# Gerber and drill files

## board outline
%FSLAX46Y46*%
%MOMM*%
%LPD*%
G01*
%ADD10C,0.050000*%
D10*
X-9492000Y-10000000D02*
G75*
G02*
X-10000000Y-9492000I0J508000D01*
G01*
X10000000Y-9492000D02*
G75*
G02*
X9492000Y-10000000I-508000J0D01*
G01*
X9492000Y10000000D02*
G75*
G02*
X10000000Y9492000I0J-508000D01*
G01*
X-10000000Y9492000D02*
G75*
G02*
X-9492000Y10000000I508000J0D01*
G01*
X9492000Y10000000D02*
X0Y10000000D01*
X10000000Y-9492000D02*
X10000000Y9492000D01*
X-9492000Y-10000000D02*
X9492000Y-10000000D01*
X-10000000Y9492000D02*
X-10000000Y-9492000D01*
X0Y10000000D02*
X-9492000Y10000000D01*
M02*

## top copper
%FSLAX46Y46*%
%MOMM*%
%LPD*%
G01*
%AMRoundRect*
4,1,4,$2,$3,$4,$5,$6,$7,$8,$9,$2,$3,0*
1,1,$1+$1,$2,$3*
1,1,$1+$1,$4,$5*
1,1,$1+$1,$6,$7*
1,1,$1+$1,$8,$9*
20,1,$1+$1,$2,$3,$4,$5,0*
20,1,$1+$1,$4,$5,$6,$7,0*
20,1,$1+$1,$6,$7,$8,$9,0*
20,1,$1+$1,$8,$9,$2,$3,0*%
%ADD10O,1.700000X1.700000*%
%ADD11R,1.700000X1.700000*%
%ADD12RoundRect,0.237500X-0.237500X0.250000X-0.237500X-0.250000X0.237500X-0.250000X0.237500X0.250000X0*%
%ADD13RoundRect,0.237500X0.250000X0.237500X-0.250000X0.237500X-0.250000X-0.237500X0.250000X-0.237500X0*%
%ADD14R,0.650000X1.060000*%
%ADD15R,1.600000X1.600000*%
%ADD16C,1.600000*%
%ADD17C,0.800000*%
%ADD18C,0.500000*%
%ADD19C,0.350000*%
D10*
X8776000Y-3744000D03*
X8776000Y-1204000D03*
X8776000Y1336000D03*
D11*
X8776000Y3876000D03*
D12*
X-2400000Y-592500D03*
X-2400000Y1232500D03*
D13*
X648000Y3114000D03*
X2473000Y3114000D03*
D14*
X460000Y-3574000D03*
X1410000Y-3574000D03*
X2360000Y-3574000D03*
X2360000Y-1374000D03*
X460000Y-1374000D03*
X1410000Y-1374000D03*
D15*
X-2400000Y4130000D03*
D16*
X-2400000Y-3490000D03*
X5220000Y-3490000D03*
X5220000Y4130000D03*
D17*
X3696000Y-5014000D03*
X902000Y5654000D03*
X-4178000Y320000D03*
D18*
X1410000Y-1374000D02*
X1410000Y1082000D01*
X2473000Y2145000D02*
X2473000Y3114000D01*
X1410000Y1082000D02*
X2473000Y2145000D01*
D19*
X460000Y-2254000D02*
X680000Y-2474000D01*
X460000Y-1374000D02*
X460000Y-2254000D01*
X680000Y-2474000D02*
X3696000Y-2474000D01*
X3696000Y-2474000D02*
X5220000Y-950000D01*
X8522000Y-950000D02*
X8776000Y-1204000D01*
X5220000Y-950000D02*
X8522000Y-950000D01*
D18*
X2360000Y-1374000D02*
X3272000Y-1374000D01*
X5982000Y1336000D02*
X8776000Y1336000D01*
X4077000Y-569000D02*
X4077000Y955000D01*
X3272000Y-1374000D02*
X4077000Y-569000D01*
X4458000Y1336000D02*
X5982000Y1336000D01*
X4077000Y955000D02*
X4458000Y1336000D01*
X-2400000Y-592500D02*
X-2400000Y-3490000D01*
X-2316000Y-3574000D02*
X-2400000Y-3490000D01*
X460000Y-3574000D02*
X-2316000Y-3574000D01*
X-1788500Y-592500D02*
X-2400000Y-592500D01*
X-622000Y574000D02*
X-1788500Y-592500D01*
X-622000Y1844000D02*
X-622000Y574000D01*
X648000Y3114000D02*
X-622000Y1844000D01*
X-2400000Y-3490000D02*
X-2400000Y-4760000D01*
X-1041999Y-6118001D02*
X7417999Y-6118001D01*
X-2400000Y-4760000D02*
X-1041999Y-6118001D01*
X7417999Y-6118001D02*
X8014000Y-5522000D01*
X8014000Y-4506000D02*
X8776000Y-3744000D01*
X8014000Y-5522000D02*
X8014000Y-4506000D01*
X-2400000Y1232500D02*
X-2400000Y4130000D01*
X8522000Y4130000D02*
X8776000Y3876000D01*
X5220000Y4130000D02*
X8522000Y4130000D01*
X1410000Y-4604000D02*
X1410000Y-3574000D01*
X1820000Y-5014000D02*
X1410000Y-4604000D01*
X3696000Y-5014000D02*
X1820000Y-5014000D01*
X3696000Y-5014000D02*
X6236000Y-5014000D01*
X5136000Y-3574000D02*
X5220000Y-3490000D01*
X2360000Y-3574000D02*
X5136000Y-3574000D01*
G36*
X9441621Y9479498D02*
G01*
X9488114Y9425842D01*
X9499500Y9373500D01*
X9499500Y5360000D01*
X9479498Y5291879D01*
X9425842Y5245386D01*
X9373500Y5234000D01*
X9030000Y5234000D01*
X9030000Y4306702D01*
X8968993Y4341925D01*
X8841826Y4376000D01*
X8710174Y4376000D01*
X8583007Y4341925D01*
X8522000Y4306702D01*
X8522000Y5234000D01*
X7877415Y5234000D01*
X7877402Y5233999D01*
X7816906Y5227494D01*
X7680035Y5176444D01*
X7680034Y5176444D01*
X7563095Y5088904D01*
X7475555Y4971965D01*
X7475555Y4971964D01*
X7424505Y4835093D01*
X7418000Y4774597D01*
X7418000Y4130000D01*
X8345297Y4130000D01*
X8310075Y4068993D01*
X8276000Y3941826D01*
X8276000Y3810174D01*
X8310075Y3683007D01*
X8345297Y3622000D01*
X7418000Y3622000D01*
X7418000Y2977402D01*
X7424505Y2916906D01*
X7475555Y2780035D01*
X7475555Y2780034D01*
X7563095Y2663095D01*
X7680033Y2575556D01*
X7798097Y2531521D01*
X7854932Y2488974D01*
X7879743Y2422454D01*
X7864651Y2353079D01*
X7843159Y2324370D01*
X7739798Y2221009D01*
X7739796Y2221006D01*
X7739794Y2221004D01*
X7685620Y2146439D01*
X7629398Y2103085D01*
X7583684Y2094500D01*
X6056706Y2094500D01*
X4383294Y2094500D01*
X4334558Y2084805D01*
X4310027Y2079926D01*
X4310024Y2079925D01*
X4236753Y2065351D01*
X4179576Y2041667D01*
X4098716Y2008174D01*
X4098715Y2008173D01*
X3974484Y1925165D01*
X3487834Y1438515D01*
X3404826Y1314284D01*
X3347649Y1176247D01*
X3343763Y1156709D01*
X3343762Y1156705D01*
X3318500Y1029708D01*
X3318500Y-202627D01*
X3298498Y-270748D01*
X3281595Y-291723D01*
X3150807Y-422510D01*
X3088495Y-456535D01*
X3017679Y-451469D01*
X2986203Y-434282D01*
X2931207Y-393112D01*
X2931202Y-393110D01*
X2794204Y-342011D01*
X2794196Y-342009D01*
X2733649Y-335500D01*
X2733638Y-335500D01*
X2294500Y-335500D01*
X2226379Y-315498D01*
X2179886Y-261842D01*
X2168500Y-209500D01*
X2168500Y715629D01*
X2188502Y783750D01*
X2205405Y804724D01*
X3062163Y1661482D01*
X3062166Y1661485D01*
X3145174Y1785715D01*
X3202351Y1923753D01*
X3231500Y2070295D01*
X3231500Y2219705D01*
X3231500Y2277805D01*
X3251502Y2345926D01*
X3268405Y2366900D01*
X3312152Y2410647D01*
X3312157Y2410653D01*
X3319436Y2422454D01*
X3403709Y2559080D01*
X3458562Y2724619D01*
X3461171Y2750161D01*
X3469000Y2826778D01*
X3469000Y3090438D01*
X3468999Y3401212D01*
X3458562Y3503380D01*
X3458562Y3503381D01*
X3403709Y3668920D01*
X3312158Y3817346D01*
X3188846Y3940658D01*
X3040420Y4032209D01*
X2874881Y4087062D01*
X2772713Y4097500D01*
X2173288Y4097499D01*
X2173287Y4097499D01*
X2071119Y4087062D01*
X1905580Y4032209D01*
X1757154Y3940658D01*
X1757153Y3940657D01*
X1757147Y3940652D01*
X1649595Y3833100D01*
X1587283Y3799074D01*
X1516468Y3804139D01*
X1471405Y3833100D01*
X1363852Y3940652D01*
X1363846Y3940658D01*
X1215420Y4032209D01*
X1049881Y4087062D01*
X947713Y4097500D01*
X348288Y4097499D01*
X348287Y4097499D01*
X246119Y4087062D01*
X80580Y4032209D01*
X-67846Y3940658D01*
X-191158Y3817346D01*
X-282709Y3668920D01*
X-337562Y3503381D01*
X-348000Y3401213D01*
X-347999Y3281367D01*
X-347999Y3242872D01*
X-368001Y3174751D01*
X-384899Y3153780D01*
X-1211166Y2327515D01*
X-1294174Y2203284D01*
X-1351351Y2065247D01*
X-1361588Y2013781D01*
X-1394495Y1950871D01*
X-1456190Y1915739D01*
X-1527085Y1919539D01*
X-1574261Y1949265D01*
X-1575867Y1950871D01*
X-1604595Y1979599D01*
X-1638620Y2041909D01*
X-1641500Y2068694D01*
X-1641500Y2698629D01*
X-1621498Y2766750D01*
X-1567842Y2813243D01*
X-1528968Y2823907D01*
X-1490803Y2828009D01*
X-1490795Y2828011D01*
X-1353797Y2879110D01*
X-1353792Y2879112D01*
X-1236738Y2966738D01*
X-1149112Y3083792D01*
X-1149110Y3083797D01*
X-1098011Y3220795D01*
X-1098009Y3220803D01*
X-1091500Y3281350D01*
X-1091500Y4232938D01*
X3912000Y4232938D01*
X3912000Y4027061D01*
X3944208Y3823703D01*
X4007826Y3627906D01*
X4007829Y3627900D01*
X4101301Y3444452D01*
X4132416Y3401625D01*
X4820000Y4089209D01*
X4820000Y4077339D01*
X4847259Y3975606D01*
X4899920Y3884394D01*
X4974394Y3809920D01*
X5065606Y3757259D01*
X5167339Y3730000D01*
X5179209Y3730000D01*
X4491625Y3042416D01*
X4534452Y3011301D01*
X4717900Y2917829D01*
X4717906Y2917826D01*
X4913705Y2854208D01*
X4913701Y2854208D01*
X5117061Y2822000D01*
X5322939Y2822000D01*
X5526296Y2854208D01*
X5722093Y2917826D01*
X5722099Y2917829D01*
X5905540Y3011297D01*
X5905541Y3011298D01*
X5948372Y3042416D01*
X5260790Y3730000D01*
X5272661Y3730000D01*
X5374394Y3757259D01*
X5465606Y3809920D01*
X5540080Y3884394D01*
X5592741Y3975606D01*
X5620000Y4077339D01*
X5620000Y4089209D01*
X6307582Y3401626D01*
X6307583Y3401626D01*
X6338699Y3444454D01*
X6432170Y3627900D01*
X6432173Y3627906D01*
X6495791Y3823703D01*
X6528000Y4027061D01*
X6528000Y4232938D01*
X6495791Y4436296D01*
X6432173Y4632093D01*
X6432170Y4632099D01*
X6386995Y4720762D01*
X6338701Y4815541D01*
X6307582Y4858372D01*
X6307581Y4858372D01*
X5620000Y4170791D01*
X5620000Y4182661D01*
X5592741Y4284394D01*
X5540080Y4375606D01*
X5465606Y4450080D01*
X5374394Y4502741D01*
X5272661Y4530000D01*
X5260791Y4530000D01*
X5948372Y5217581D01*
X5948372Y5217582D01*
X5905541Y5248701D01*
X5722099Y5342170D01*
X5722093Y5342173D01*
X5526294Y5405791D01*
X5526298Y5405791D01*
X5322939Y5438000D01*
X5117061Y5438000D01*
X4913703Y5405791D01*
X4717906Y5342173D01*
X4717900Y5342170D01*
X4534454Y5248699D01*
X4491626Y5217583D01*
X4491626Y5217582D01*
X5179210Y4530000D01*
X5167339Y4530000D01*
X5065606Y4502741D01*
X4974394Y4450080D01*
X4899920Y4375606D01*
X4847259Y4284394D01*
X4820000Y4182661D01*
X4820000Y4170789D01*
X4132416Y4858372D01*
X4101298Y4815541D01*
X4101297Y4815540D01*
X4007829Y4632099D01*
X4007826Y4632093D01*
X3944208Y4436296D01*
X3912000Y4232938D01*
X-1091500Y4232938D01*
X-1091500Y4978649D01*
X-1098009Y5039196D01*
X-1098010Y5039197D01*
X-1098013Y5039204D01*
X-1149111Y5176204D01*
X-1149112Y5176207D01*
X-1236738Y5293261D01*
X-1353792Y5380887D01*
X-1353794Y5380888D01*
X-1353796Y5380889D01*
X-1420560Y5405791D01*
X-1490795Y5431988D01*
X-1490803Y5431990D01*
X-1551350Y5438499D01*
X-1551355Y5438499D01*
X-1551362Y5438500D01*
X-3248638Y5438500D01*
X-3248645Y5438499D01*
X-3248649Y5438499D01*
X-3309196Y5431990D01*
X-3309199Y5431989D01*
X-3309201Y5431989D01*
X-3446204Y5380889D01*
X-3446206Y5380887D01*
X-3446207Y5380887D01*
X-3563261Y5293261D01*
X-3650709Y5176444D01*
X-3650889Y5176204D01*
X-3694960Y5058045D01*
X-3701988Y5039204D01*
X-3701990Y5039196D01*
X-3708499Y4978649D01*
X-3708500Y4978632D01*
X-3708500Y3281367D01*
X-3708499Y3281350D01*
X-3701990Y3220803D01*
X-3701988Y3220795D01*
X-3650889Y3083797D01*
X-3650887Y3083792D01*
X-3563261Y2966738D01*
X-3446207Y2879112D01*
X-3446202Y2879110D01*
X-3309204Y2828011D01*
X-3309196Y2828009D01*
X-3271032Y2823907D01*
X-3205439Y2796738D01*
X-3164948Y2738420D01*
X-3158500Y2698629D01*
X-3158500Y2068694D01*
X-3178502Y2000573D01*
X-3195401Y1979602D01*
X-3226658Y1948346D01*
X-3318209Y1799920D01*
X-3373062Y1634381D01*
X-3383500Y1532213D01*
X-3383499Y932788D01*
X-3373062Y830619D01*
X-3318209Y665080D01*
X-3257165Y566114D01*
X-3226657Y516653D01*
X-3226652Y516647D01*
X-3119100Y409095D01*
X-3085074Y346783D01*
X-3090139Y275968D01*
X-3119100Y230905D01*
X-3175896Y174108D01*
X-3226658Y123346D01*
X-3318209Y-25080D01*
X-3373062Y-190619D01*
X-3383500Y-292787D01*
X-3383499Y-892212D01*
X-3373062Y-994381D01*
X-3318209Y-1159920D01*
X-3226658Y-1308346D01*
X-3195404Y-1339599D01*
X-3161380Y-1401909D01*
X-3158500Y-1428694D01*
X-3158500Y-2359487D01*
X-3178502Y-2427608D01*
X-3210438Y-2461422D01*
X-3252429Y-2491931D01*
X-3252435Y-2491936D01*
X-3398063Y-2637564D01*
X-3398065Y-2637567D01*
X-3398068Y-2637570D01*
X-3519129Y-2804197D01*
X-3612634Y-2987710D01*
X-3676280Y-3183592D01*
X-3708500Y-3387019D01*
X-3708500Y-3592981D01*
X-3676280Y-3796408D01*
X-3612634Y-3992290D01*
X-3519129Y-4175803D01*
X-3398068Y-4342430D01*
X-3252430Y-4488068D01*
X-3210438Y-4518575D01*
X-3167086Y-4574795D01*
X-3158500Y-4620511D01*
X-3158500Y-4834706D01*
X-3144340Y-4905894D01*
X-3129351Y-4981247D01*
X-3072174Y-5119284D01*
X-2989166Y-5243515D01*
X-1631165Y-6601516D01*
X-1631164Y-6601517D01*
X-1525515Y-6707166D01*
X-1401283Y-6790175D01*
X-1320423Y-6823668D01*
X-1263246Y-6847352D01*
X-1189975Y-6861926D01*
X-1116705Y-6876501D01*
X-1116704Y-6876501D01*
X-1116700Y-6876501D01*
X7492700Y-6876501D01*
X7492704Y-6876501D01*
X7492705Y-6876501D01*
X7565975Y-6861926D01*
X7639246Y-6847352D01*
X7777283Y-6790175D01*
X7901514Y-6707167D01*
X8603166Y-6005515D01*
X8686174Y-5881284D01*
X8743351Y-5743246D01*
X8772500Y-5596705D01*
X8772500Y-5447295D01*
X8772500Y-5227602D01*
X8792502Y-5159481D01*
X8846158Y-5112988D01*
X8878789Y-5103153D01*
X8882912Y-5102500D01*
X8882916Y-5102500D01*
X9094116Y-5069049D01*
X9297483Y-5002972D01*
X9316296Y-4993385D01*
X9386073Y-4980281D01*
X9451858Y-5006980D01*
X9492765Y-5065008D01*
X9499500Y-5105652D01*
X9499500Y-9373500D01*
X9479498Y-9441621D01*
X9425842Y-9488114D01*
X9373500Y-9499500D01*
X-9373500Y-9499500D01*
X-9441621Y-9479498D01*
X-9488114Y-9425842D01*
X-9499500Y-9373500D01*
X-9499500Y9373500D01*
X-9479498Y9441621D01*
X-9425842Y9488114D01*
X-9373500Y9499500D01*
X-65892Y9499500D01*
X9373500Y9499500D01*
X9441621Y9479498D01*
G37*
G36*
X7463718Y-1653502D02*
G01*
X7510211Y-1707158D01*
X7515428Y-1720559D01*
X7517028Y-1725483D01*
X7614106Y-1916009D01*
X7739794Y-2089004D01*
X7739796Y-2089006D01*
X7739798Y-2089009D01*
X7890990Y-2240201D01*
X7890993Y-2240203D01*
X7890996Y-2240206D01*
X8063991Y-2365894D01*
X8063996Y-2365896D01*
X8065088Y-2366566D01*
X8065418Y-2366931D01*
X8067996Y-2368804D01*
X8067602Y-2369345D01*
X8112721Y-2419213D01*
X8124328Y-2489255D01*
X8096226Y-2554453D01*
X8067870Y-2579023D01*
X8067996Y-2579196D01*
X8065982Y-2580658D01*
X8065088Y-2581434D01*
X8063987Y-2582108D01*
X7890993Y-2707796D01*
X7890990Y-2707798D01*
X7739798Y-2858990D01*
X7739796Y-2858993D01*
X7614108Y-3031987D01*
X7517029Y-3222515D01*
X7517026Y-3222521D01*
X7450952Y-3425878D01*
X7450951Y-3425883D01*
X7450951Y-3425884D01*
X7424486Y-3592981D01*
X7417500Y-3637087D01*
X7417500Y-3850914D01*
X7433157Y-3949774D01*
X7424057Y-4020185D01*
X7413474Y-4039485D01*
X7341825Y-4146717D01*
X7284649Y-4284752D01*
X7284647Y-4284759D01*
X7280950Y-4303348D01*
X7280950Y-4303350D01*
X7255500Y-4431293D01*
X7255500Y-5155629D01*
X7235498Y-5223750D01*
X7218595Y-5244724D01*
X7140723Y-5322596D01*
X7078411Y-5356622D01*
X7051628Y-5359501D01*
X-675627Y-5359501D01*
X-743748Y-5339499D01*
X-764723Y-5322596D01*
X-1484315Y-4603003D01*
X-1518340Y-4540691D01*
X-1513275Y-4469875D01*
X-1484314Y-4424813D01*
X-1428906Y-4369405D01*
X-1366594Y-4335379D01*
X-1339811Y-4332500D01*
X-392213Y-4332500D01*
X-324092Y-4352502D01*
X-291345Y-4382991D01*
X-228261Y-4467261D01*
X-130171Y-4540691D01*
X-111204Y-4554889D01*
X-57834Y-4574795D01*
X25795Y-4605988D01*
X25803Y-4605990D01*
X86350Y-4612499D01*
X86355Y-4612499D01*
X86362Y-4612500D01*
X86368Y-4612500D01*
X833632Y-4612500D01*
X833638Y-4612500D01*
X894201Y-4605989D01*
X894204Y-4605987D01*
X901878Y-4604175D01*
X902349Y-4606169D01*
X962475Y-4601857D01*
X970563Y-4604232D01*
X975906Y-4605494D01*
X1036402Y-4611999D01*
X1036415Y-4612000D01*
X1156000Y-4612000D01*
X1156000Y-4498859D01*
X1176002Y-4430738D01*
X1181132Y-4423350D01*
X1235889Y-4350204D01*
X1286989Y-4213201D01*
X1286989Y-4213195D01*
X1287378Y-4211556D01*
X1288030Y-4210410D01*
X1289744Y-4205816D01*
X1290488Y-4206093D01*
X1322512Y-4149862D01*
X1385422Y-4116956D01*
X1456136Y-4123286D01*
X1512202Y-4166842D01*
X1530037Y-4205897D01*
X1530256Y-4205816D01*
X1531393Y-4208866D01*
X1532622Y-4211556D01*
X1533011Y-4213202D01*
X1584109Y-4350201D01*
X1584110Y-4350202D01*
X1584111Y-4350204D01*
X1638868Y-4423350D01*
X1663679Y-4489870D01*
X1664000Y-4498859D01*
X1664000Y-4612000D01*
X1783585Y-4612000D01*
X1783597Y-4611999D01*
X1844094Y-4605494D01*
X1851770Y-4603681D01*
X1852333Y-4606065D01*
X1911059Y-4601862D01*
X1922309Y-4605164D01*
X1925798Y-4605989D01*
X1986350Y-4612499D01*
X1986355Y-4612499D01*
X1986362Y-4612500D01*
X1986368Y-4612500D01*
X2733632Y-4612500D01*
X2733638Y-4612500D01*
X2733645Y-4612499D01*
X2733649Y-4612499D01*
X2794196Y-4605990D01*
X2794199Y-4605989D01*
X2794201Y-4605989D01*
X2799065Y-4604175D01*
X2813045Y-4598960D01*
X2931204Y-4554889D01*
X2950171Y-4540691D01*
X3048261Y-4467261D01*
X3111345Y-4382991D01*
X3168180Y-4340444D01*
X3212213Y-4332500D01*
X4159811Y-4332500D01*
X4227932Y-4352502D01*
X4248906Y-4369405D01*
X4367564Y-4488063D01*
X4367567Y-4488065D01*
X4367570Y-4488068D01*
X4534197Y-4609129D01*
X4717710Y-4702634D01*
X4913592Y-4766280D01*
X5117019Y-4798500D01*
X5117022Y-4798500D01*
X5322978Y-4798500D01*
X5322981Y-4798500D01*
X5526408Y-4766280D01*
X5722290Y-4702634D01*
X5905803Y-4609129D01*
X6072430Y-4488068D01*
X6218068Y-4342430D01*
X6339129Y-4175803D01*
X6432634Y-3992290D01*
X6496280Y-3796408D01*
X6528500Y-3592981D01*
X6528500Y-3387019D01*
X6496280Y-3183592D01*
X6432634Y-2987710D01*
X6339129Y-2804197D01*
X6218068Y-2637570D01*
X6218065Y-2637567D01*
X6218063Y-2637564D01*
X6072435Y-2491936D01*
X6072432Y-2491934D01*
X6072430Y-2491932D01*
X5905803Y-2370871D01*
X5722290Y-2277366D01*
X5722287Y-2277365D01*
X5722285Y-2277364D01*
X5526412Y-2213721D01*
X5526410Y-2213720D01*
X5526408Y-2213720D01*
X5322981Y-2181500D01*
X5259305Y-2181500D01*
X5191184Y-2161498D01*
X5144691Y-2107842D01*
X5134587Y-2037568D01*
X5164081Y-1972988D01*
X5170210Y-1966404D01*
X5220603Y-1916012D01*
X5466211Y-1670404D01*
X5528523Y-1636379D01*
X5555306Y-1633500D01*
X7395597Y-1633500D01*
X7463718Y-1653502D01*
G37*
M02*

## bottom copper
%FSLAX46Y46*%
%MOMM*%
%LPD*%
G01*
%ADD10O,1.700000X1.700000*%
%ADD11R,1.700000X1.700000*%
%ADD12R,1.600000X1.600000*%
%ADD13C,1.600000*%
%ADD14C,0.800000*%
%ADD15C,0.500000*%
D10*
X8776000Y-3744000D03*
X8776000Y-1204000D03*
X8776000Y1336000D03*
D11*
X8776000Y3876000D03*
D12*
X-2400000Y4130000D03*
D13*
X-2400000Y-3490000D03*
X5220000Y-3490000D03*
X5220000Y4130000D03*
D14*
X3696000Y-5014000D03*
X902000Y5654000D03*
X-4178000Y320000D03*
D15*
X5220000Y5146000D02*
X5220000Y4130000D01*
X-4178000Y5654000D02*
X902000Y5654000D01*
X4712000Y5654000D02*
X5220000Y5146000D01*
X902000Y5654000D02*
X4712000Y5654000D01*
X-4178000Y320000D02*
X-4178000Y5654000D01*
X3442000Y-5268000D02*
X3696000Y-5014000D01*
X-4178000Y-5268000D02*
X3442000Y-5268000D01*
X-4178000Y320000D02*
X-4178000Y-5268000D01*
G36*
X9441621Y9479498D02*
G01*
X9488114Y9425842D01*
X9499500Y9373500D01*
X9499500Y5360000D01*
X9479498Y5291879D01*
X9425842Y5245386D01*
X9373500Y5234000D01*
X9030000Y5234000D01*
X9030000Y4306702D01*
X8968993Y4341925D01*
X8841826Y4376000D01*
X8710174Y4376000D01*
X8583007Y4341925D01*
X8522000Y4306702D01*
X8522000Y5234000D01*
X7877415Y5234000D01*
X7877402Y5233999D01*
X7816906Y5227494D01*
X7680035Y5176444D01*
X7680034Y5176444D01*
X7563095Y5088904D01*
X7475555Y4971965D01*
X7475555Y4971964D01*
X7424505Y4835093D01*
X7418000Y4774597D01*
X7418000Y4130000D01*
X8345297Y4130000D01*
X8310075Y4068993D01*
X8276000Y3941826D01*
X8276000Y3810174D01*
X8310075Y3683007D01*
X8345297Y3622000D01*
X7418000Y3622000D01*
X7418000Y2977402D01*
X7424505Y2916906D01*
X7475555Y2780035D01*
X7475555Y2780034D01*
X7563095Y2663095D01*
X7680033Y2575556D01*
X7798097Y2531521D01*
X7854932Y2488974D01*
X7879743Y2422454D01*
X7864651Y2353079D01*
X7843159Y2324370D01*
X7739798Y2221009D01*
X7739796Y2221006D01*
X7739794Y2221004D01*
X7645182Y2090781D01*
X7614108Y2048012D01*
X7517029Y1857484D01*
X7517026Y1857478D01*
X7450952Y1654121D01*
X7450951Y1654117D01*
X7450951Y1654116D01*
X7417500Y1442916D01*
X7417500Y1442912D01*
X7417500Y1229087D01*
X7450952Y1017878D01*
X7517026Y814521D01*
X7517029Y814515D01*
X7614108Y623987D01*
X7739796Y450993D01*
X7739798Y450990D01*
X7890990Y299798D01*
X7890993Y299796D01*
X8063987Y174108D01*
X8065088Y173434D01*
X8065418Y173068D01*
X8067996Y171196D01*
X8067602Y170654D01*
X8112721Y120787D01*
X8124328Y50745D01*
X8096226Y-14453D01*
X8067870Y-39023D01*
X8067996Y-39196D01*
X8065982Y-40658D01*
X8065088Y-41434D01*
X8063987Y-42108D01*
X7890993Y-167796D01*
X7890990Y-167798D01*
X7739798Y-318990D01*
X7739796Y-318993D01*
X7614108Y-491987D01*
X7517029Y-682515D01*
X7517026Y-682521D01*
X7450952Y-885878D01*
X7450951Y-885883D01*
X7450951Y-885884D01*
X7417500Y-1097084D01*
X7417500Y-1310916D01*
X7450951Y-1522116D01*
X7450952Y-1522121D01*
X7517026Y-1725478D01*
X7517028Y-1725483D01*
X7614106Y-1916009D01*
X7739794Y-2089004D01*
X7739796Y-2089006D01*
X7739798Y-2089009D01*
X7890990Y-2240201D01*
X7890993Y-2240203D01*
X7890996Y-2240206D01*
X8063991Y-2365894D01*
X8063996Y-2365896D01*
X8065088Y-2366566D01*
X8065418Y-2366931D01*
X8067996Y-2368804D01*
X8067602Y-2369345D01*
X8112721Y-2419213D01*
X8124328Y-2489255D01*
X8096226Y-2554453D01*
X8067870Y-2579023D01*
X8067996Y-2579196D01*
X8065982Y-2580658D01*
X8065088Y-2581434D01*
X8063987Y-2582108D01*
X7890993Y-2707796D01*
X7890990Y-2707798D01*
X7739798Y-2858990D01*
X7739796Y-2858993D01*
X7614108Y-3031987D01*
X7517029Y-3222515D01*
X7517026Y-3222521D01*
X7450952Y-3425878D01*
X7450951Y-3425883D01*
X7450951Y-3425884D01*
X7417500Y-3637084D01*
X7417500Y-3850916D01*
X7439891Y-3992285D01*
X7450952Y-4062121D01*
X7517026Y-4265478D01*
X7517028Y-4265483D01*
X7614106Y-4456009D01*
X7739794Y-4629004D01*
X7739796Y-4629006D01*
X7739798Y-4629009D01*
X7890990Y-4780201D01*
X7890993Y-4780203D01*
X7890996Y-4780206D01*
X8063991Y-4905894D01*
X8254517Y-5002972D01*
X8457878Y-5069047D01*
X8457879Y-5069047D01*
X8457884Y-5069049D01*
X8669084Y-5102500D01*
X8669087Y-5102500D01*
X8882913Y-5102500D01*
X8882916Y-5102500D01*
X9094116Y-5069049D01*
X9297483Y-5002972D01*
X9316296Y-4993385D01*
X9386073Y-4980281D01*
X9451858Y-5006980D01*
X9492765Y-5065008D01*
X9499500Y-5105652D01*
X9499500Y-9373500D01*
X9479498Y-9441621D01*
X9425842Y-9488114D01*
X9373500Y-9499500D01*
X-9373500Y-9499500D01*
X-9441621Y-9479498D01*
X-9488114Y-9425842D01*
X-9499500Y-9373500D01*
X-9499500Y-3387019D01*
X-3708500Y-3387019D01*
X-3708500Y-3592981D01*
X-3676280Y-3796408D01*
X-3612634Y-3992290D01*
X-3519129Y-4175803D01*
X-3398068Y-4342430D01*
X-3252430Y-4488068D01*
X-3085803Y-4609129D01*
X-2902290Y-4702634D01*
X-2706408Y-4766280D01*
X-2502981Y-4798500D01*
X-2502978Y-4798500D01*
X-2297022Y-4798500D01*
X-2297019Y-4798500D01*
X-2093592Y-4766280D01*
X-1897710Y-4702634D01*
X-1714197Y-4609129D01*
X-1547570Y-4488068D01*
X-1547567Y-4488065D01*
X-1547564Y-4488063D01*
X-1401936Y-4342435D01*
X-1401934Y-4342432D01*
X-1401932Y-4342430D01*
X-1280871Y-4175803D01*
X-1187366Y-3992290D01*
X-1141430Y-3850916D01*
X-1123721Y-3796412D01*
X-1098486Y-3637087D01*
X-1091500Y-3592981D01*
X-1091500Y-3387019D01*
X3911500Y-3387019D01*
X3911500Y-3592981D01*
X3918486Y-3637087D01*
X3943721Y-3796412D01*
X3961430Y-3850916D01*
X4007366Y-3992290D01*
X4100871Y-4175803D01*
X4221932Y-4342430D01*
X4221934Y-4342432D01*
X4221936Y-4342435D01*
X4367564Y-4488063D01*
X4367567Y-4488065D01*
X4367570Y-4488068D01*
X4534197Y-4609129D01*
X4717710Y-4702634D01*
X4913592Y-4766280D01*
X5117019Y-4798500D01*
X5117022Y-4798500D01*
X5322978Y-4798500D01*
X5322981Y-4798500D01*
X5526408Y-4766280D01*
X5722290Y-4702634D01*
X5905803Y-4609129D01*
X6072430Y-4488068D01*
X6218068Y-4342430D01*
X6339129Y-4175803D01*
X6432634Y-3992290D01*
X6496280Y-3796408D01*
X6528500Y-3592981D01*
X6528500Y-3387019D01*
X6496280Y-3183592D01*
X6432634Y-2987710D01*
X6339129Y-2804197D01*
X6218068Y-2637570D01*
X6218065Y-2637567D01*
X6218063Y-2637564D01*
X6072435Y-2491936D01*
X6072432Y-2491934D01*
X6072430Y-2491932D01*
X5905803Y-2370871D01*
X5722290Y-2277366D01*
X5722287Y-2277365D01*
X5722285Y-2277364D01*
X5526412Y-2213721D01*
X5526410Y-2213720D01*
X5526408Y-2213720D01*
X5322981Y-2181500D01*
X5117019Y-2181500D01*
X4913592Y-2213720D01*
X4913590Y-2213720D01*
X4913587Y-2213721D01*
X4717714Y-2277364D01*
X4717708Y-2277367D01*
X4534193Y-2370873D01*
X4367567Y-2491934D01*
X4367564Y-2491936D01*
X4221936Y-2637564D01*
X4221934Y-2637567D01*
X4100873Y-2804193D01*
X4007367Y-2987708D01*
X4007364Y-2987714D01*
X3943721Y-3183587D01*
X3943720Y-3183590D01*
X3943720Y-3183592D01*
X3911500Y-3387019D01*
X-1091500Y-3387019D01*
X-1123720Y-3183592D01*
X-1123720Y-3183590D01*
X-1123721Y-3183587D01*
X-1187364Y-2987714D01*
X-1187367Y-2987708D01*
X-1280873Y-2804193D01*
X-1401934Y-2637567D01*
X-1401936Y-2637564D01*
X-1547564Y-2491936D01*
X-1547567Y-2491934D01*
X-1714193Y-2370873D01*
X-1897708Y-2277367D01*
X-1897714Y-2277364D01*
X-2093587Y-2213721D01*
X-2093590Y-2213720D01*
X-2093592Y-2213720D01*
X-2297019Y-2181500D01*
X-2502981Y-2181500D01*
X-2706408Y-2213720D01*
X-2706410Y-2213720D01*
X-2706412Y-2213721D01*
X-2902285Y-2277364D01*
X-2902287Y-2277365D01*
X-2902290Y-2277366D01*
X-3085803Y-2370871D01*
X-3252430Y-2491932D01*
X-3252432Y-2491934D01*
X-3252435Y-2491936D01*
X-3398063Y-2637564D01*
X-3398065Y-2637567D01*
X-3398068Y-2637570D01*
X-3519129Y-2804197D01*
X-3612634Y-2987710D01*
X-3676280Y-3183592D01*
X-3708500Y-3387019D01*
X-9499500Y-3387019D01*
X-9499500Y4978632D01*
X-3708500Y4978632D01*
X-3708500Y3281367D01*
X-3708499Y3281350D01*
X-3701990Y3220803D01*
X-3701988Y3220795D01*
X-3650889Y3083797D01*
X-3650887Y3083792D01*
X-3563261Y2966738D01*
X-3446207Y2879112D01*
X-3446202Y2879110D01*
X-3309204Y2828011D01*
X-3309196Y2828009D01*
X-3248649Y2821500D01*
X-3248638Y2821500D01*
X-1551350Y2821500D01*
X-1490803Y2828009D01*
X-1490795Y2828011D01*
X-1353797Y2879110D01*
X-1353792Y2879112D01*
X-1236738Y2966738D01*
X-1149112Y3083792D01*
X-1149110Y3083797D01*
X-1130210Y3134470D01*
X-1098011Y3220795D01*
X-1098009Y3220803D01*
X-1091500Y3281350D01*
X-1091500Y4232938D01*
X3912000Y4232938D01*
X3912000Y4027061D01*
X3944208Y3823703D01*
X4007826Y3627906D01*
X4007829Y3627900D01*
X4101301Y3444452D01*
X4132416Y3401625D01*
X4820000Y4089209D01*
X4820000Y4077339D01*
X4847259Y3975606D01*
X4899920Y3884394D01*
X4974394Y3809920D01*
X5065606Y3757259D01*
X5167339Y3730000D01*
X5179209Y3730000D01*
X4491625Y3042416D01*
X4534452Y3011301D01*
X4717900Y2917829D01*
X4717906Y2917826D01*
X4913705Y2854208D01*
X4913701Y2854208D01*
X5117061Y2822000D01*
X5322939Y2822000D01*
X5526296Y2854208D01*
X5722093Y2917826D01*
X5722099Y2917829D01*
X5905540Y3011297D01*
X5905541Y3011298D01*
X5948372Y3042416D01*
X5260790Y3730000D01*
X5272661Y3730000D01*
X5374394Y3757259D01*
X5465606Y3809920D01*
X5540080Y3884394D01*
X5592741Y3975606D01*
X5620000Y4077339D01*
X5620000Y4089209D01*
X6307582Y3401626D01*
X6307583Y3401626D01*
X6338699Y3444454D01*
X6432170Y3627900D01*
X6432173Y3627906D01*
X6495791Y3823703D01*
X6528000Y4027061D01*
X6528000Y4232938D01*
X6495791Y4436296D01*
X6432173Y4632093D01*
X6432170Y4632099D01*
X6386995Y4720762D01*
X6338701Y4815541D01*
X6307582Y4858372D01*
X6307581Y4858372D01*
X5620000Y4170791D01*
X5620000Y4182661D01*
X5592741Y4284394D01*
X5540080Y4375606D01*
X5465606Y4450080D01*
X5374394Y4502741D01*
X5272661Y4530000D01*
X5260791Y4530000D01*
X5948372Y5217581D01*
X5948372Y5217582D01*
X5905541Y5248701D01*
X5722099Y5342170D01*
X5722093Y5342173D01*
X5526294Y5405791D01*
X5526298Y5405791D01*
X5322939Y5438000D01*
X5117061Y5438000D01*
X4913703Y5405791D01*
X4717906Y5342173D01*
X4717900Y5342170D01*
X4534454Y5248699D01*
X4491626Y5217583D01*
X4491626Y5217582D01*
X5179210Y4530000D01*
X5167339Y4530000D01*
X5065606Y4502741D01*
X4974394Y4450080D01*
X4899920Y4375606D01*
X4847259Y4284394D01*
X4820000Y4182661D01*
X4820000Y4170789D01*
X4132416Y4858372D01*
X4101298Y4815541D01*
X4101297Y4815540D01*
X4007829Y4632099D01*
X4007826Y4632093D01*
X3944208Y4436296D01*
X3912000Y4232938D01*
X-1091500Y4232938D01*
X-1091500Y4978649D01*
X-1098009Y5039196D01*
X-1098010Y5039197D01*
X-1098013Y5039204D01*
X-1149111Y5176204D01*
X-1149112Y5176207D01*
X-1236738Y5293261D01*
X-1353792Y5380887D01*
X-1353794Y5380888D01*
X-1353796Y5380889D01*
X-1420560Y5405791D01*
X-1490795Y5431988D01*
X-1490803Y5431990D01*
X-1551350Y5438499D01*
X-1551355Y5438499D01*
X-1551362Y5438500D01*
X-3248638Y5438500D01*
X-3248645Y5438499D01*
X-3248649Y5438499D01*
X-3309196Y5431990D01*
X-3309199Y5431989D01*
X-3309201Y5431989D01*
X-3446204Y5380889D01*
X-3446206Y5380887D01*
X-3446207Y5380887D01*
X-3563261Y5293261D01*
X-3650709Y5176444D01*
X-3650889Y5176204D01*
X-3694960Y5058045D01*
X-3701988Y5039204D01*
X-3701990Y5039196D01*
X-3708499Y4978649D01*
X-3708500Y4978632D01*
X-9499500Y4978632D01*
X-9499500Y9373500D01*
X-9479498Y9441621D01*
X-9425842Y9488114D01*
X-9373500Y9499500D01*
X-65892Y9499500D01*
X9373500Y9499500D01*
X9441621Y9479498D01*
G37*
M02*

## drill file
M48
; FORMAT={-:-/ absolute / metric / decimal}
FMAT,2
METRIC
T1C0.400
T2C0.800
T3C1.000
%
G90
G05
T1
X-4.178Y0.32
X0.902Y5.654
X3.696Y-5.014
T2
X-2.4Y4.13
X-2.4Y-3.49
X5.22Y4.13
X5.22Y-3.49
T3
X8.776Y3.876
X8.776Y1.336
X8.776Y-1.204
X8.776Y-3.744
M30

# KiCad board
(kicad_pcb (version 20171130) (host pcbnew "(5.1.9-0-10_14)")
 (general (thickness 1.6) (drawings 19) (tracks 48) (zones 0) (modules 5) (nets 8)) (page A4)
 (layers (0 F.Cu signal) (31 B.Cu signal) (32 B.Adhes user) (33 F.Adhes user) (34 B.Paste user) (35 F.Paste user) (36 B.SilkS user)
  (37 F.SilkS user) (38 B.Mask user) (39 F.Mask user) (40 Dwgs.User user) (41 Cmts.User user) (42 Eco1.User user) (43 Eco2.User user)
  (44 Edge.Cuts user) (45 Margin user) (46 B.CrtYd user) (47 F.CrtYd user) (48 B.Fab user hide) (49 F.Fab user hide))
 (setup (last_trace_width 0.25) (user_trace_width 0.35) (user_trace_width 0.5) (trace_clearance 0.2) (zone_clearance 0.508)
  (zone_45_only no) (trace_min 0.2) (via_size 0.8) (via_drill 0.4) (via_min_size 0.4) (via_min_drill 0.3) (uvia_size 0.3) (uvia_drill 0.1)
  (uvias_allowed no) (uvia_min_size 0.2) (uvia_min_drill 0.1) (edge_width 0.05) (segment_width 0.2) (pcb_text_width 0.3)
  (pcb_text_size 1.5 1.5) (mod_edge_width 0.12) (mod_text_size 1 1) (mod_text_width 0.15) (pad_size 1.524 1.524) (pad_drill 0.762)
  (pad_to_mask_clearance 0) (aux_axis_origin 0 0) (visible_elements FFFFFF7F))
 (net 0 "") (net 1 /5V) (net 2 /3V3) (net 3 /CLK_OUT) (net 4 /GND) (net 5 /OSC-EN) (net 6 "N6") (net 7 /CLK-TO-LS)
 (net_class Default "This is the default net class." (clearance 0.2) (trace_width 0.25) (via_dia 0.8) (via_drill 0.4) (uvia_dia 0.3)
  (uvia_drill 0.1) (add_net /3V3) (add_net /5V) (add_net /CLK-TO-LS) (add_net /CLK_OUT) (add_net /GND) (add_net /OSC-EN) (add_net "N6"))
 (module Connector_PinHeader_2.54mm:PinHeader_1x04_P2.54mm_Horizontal (layer F.Cu) (at 8.776 -3.876)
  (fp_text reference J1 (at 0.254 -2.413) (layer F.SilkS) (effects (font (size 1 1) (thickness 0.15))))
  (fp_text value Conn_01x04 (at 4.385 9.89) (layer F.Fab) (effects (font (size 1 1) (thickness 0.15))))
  (pad 4 thru_hole oval (at 0 7.62) (size 1.7 1.7) (drill 1) (layers *.Cu *.Mask) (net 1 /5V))
  (pad 3 thru_hole oval (at 0 5.08) (size 1.7 1.7) (drill 1) (layers *.Cu *.Mask) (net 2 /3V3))
  (pad 2 thru_hole oval (at 0 2.54) (size 1.7 1.7) (drill 1) (layers *.Cu *.Mask) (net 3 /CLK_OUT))
  (pad 1 thru_hole rect (at 0 0) (size 1.7 1.7) (drill 1) (layers *.Cu *.Mask) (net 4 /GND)))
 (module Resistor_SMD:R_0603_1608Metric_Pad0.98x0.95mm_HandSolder (layer F.Cu) (at -2.4 -0.32 270)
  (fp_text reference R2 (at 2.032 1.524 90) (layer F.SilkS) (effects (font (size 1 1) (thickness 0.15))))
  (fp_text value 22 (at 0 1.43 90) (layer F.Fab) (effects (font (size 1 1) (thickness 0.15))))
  (pad 2 smd roundrect (at 0.9125 0 270) (size 0.975 0.95) (layers F.Cu F.Paste F.Mask) (roundrect_rratio 0.25) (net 1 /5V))
  (pad 1 smd roundrect (at -0.9125 0 270) (size 0.975 0.95) (layers F.Cu F.Paste F.Mask) (roundrect_rratio 0.25) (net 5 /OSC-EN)))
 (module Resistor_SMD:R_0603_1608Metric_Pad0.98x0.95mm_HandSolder (layer F.Cu) (at 1.5605 -3.114 180)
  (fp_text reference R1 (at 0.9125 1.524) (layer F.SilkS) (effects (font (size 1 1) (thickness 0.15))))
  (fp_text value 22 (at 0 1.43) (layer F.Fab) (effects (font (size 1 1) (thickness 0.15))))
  (pad 2 smd roundrect (at 0.9125 0 180) (size 0.975 0.95) (layers F.Cu F.Paste F.Mask) (roundrect_rratio 0.25) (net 1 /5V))
  (pad 1 smd roundrect (at -0.9125 0 180) (size 0.975 0.95) (layers F.Cu F.Paste F.Mask) (roundrect_rratio 0.25) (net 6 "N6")))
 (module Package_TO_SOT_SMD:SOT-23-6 (layer F.Cu) (at 1.41 2.474 90)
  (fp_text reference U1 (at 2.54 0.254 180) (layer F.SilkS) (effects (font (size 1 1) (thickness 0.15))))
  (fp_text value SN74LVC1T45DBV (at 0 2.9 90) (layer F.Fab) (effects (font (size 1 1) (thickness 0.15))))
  (pad 1 smd rect (at -1.1 -0.95 90) (size 1.06 0.65) (layers F.Cu F.Paste F.Mask) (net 1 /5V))
  (pad 2 smd rect (at -1.1 0 90) (size 1.06 0.65) (layers F.Cu F.Paste F.Mask) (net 4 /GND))
  (pad 3 smd rect (at -1.1 0.95 90) (size 1.06 0.65) (layers F.Cu F.Paste F.Mask) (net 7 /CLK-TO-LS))
  (pad 4 smd rect (at 1.1 0.95 90) (size 1.06 0.65) (layers F.Cu F.Paste F.Mask) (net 3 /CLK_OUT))
  (pad 6 smd rect (at 1.1 -0.95 90) (size 1.06 0.65) (layers F.Cu F.Paste F.Mask) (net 2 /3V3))
  (pad 5 smd rect (at 1.1 0 90) (size 1.06 0.65) (layers F.Cu F.Paste F.Mask) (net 6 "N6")))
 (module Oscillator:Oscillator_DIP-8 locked (layer B.Cu) (at -2.4 -4.13)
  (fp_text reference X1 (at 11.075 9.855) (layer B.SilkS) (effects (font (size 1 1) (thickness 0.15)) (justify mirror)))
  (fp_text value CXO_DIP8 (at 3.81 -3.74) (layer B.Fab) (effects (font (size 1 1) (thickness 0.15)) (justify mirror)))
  (pad 1 thru_hole rect (at 0 0) (size 1.6 1.6) (drill 0.8) (layers *.Cu *.Mask) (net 5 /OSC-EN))
  (pad 8 thru_hole circle (at 0 7.62) (size 1.6 1.6) (drill 0.8) (layers *.Cu *.Mask) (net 1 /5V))
  (pad 5 thru_hole circle (at 7.62 7.62) (size 1.6 1.6) (drill 0.8) (layers *.Cu *.Mask) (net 7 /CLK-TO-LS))
  (pad 4 thru_hole circle (at 7.62 0) (size 1.6 1.6) (drill 0.8) (layers *.Cu *.Mask) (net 4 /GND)))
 (gr_arc (start -9.492 9.492) (end -10 9.492) (angle -90) (layer Edge.Cuts) (width 0.05))
 (gr_arc (start 9.492 9.492) (end 9.492 10) (angle -90) (layer Edge.Cuts) (width 0.05))
 (gr_arc (start 9.492 -9.492) (end 10 -9.492) (angle -90) (layer Edge.Cuts) (width 0.05))
 (gr_arc (start -9.492 -9.492) (end -9.492 -10) (angle -90) (layer Edge.Cuts) (width 0.05))
 (gr_line (start 9.492 -10) (end 0 -10) (layer Edge.Cuts) (width 0.05))
 (gr_line (start 10 9.492) (end 10 -9.492) (layer Edge.Cuts) (width 0.05))
 (gr_line (start -9.492 10) (end 9.492 10) (layer Edge.Cuts) (width 0.05))
 (gr_line (start -10 -9.492) (end -10 9.492) (layer Edge.Cuts) (width 0.05))
 (gr_line (start 0 -10) (end -9.492 -10) (layer Edge.Cuts) (width 0.05))
 (segment (start 1.41 1.374) (end 1.41 -1.082) (width 0.5) (layer F.Cu) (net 6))
 (segment (start 2.473 -2.145) (end 2.473 -3.114) (width 0.5) (layer F.Cu) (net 6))
 (segment (start 1.41 -1.082) (end 2.473 -2.145) (width 0.5) (layer F.Cu) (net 6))
 (segment (start 0.46 2.254) (end 0.68 2.474) (width 0.35) (layer F.Cu) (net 2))
 (segment (start 0.46 1.374) (end 0.46 2.254) (width 0.35) (layer F.Cu) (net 2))
 (segment (start 0.68 2.474) (end 3.696 2.474) (width 0.35) (layer F.Cu) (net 2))
 (segment (start 3.696 2.474) (end 5.22 0.95) (width 0.35) (layer F.Cu) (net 2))
 (segment (start 8.522 0.95) (end 8.776 1.204) (width 0.35) (layer F.Cu) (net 2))
 (segment (start 5.22 0.95) (end 8.522 0.95) (width 0.35) (layer F.Cu) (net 2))
 (segment (start 2.36 1.374) (end 3.272 1.374) (width 0.5) (layer F.Cu) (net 3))
 (segment (start 5.982 -1.336) (end 8.776 -1.336) (width 0.5) (layer F.Cu) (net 3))
 (segment (start 4.077 0.569) (end 4.077 -0.955) (width 0.5) (layer F.Cu) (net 3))
 (segment (start 3.272 1.374) (end 4.077 0.569) (width 0.5) (layer F.Cu) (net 3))
 (segment (start 4.458 -1.336) (end 5.982 -1.336) (width 0.5) (layer F.Cu) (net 3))
 (segment (start 4.077 -0.955) (end 4.458 -1.336) (width 0.5) (layer F.Cu) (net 3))
 (segment (start -2.4 0.5925) (end -2.4 3.49) (width 0.5) (layer F.Cu) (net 1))
 (segment (start -2.316 3.574) (end -2.4 3.49) (width 0.5) (layer F.Cu) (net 1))
 (segment (start 0.46 3.574) (end -2.316 3.574) (width 0.5) (layer F.Cu) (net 1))
 (segment (start -1.7885 0.5925) (end -2.4 0.5925) (width 0.5) (layer F.Cu) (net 1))
 (segment (start -0.622 -0.574) (end -1.7885 0.5925) (width 0.5) (layer F.Cu) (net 1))
 (segment (start -0.622 -1.844) (end -0.622 -0.574) (width 0.5) (layer F.Cu) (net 1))
 (segment (start 0.648 -3.114) (end -0.622 -1.844) (width 0.5) (layer F.Cu) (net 1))
 (segment (start -2.4 3.49) (end -2.4 4.76) (width 0.5) (layer F.Cu) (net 1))
 (segment (start -1.041999 6.118001) (end 7.417999 6.118001) (width 0.5) (layer F.Cu) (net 1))
 (segment (start -2.4 4.76) (end -1.041999 6.118001) (width 0.5) (layer F.Cu) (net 1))
 (segment (start 7.417999 6.118001) (end 8.014 5.522) (width 0.5) (layer F.Cu) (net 1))
 (segment (start 8.014 4.506) (end 8.776 3.744) (width 0.5) (layer F.Cu) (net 1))
 (segment (start 8.014 5.522) (end 8.014 4.506) (width 0.5) (layer F.Cu) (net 1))
 (segment (start -2.4 -1.2325) (end -2.4 -4.13) (width 0.5) (layer F.Cu) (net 5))
 (via (at 3.696 5.014) (size 0.8) (drill 0.4) (layers F.Cu B.Cu) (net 4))
 (segment (start 5.22 -5.146) (end 5.22 -4.13) (width 0.5) (layer B.Cu) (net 4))
 (segment (start -4.178 -5.654) (end 0.902 -5.654) (width 0.5) (layer B.Cu) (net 4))
 (segment (start 4.712 -5.654) (end 5.22 -5.146) (width 0.5) (layer B.Cu) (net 4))
 (segment (start 8.522 -4.13) (end 8.776 -3.876) (width 0.5) (layer F.Cu) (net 4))
 (segment (start 5.22 -4.13) (end 8.522 -4.13) (width 0.5) (layer F.Cu) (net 4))
 (segment (start 0.902 -5.654) (end 4.712 -5.654) (width 0.5) (layer B.Cu) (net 4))
 (via (at 0.902 -5.654) (size 0.8) (drill 0.4) (layers F.Cu B.Cu) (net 4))
 (segment (start -4.178 -0.32) (end -4.178 -5.654) (width 0.5) (layer B.Cu) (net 4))
 (via (at -4.178 -0.32) (size 0.8) (drill 0.4) (layers F.Cu B.Cu) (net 4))
 (segment (start 1.41 4.604) (end 1.41 3.574) (width 0.5) (layer F.Cu) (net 4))
 (segment (start 1.82 5.014) (end 1.41 4.604) (width 0.5) (layer F.Cu) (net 4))
 (segment (start 3.696 5.014) (end 1.82 5.014) (width 0.5) (layer F.Cu) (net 4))
 (segment (start 3.442 5.268) (end 3.696 5.014) (width 0.5) (layer B.Cu) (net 4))
 (segment (start -4.178 5.268) (end 3.442 5.268) (width 0.5) (layer B.Cu) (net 4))
 (segment (start -4.178 -0.32) (end -4.178 5.268) (width 0.5) (layer B.Cu) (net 4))
 (segment (start 3.696 5.014) (end 6.236 5.014) (width 0.5) (layer F.Cu) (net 4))
 (segment (start 5.136 3.574) (end 5.22 3.49) (width 0.5) (layer F.Cu) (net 7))
 (segment (start 2.36 3.574) (end 5.136 3.574) (width 0.5) (layer F.Cu) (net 7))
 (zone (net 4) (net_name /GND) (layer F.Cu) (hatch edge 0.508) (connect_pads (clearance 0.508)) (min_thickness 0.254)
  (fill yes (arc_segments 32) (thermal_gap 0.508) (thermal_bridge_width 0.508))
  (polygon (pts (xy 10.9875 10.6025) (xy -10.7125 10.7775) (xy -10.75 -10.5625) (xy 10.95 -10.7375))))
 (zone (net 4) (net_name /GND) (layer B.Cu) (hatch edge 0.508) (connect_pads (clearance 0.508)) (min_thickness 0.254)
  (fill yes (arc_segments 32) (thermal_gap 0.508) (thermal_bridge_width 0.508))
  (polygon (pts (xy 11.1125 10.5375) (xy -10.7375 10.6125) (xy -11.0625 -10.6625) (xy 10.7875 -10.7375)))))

